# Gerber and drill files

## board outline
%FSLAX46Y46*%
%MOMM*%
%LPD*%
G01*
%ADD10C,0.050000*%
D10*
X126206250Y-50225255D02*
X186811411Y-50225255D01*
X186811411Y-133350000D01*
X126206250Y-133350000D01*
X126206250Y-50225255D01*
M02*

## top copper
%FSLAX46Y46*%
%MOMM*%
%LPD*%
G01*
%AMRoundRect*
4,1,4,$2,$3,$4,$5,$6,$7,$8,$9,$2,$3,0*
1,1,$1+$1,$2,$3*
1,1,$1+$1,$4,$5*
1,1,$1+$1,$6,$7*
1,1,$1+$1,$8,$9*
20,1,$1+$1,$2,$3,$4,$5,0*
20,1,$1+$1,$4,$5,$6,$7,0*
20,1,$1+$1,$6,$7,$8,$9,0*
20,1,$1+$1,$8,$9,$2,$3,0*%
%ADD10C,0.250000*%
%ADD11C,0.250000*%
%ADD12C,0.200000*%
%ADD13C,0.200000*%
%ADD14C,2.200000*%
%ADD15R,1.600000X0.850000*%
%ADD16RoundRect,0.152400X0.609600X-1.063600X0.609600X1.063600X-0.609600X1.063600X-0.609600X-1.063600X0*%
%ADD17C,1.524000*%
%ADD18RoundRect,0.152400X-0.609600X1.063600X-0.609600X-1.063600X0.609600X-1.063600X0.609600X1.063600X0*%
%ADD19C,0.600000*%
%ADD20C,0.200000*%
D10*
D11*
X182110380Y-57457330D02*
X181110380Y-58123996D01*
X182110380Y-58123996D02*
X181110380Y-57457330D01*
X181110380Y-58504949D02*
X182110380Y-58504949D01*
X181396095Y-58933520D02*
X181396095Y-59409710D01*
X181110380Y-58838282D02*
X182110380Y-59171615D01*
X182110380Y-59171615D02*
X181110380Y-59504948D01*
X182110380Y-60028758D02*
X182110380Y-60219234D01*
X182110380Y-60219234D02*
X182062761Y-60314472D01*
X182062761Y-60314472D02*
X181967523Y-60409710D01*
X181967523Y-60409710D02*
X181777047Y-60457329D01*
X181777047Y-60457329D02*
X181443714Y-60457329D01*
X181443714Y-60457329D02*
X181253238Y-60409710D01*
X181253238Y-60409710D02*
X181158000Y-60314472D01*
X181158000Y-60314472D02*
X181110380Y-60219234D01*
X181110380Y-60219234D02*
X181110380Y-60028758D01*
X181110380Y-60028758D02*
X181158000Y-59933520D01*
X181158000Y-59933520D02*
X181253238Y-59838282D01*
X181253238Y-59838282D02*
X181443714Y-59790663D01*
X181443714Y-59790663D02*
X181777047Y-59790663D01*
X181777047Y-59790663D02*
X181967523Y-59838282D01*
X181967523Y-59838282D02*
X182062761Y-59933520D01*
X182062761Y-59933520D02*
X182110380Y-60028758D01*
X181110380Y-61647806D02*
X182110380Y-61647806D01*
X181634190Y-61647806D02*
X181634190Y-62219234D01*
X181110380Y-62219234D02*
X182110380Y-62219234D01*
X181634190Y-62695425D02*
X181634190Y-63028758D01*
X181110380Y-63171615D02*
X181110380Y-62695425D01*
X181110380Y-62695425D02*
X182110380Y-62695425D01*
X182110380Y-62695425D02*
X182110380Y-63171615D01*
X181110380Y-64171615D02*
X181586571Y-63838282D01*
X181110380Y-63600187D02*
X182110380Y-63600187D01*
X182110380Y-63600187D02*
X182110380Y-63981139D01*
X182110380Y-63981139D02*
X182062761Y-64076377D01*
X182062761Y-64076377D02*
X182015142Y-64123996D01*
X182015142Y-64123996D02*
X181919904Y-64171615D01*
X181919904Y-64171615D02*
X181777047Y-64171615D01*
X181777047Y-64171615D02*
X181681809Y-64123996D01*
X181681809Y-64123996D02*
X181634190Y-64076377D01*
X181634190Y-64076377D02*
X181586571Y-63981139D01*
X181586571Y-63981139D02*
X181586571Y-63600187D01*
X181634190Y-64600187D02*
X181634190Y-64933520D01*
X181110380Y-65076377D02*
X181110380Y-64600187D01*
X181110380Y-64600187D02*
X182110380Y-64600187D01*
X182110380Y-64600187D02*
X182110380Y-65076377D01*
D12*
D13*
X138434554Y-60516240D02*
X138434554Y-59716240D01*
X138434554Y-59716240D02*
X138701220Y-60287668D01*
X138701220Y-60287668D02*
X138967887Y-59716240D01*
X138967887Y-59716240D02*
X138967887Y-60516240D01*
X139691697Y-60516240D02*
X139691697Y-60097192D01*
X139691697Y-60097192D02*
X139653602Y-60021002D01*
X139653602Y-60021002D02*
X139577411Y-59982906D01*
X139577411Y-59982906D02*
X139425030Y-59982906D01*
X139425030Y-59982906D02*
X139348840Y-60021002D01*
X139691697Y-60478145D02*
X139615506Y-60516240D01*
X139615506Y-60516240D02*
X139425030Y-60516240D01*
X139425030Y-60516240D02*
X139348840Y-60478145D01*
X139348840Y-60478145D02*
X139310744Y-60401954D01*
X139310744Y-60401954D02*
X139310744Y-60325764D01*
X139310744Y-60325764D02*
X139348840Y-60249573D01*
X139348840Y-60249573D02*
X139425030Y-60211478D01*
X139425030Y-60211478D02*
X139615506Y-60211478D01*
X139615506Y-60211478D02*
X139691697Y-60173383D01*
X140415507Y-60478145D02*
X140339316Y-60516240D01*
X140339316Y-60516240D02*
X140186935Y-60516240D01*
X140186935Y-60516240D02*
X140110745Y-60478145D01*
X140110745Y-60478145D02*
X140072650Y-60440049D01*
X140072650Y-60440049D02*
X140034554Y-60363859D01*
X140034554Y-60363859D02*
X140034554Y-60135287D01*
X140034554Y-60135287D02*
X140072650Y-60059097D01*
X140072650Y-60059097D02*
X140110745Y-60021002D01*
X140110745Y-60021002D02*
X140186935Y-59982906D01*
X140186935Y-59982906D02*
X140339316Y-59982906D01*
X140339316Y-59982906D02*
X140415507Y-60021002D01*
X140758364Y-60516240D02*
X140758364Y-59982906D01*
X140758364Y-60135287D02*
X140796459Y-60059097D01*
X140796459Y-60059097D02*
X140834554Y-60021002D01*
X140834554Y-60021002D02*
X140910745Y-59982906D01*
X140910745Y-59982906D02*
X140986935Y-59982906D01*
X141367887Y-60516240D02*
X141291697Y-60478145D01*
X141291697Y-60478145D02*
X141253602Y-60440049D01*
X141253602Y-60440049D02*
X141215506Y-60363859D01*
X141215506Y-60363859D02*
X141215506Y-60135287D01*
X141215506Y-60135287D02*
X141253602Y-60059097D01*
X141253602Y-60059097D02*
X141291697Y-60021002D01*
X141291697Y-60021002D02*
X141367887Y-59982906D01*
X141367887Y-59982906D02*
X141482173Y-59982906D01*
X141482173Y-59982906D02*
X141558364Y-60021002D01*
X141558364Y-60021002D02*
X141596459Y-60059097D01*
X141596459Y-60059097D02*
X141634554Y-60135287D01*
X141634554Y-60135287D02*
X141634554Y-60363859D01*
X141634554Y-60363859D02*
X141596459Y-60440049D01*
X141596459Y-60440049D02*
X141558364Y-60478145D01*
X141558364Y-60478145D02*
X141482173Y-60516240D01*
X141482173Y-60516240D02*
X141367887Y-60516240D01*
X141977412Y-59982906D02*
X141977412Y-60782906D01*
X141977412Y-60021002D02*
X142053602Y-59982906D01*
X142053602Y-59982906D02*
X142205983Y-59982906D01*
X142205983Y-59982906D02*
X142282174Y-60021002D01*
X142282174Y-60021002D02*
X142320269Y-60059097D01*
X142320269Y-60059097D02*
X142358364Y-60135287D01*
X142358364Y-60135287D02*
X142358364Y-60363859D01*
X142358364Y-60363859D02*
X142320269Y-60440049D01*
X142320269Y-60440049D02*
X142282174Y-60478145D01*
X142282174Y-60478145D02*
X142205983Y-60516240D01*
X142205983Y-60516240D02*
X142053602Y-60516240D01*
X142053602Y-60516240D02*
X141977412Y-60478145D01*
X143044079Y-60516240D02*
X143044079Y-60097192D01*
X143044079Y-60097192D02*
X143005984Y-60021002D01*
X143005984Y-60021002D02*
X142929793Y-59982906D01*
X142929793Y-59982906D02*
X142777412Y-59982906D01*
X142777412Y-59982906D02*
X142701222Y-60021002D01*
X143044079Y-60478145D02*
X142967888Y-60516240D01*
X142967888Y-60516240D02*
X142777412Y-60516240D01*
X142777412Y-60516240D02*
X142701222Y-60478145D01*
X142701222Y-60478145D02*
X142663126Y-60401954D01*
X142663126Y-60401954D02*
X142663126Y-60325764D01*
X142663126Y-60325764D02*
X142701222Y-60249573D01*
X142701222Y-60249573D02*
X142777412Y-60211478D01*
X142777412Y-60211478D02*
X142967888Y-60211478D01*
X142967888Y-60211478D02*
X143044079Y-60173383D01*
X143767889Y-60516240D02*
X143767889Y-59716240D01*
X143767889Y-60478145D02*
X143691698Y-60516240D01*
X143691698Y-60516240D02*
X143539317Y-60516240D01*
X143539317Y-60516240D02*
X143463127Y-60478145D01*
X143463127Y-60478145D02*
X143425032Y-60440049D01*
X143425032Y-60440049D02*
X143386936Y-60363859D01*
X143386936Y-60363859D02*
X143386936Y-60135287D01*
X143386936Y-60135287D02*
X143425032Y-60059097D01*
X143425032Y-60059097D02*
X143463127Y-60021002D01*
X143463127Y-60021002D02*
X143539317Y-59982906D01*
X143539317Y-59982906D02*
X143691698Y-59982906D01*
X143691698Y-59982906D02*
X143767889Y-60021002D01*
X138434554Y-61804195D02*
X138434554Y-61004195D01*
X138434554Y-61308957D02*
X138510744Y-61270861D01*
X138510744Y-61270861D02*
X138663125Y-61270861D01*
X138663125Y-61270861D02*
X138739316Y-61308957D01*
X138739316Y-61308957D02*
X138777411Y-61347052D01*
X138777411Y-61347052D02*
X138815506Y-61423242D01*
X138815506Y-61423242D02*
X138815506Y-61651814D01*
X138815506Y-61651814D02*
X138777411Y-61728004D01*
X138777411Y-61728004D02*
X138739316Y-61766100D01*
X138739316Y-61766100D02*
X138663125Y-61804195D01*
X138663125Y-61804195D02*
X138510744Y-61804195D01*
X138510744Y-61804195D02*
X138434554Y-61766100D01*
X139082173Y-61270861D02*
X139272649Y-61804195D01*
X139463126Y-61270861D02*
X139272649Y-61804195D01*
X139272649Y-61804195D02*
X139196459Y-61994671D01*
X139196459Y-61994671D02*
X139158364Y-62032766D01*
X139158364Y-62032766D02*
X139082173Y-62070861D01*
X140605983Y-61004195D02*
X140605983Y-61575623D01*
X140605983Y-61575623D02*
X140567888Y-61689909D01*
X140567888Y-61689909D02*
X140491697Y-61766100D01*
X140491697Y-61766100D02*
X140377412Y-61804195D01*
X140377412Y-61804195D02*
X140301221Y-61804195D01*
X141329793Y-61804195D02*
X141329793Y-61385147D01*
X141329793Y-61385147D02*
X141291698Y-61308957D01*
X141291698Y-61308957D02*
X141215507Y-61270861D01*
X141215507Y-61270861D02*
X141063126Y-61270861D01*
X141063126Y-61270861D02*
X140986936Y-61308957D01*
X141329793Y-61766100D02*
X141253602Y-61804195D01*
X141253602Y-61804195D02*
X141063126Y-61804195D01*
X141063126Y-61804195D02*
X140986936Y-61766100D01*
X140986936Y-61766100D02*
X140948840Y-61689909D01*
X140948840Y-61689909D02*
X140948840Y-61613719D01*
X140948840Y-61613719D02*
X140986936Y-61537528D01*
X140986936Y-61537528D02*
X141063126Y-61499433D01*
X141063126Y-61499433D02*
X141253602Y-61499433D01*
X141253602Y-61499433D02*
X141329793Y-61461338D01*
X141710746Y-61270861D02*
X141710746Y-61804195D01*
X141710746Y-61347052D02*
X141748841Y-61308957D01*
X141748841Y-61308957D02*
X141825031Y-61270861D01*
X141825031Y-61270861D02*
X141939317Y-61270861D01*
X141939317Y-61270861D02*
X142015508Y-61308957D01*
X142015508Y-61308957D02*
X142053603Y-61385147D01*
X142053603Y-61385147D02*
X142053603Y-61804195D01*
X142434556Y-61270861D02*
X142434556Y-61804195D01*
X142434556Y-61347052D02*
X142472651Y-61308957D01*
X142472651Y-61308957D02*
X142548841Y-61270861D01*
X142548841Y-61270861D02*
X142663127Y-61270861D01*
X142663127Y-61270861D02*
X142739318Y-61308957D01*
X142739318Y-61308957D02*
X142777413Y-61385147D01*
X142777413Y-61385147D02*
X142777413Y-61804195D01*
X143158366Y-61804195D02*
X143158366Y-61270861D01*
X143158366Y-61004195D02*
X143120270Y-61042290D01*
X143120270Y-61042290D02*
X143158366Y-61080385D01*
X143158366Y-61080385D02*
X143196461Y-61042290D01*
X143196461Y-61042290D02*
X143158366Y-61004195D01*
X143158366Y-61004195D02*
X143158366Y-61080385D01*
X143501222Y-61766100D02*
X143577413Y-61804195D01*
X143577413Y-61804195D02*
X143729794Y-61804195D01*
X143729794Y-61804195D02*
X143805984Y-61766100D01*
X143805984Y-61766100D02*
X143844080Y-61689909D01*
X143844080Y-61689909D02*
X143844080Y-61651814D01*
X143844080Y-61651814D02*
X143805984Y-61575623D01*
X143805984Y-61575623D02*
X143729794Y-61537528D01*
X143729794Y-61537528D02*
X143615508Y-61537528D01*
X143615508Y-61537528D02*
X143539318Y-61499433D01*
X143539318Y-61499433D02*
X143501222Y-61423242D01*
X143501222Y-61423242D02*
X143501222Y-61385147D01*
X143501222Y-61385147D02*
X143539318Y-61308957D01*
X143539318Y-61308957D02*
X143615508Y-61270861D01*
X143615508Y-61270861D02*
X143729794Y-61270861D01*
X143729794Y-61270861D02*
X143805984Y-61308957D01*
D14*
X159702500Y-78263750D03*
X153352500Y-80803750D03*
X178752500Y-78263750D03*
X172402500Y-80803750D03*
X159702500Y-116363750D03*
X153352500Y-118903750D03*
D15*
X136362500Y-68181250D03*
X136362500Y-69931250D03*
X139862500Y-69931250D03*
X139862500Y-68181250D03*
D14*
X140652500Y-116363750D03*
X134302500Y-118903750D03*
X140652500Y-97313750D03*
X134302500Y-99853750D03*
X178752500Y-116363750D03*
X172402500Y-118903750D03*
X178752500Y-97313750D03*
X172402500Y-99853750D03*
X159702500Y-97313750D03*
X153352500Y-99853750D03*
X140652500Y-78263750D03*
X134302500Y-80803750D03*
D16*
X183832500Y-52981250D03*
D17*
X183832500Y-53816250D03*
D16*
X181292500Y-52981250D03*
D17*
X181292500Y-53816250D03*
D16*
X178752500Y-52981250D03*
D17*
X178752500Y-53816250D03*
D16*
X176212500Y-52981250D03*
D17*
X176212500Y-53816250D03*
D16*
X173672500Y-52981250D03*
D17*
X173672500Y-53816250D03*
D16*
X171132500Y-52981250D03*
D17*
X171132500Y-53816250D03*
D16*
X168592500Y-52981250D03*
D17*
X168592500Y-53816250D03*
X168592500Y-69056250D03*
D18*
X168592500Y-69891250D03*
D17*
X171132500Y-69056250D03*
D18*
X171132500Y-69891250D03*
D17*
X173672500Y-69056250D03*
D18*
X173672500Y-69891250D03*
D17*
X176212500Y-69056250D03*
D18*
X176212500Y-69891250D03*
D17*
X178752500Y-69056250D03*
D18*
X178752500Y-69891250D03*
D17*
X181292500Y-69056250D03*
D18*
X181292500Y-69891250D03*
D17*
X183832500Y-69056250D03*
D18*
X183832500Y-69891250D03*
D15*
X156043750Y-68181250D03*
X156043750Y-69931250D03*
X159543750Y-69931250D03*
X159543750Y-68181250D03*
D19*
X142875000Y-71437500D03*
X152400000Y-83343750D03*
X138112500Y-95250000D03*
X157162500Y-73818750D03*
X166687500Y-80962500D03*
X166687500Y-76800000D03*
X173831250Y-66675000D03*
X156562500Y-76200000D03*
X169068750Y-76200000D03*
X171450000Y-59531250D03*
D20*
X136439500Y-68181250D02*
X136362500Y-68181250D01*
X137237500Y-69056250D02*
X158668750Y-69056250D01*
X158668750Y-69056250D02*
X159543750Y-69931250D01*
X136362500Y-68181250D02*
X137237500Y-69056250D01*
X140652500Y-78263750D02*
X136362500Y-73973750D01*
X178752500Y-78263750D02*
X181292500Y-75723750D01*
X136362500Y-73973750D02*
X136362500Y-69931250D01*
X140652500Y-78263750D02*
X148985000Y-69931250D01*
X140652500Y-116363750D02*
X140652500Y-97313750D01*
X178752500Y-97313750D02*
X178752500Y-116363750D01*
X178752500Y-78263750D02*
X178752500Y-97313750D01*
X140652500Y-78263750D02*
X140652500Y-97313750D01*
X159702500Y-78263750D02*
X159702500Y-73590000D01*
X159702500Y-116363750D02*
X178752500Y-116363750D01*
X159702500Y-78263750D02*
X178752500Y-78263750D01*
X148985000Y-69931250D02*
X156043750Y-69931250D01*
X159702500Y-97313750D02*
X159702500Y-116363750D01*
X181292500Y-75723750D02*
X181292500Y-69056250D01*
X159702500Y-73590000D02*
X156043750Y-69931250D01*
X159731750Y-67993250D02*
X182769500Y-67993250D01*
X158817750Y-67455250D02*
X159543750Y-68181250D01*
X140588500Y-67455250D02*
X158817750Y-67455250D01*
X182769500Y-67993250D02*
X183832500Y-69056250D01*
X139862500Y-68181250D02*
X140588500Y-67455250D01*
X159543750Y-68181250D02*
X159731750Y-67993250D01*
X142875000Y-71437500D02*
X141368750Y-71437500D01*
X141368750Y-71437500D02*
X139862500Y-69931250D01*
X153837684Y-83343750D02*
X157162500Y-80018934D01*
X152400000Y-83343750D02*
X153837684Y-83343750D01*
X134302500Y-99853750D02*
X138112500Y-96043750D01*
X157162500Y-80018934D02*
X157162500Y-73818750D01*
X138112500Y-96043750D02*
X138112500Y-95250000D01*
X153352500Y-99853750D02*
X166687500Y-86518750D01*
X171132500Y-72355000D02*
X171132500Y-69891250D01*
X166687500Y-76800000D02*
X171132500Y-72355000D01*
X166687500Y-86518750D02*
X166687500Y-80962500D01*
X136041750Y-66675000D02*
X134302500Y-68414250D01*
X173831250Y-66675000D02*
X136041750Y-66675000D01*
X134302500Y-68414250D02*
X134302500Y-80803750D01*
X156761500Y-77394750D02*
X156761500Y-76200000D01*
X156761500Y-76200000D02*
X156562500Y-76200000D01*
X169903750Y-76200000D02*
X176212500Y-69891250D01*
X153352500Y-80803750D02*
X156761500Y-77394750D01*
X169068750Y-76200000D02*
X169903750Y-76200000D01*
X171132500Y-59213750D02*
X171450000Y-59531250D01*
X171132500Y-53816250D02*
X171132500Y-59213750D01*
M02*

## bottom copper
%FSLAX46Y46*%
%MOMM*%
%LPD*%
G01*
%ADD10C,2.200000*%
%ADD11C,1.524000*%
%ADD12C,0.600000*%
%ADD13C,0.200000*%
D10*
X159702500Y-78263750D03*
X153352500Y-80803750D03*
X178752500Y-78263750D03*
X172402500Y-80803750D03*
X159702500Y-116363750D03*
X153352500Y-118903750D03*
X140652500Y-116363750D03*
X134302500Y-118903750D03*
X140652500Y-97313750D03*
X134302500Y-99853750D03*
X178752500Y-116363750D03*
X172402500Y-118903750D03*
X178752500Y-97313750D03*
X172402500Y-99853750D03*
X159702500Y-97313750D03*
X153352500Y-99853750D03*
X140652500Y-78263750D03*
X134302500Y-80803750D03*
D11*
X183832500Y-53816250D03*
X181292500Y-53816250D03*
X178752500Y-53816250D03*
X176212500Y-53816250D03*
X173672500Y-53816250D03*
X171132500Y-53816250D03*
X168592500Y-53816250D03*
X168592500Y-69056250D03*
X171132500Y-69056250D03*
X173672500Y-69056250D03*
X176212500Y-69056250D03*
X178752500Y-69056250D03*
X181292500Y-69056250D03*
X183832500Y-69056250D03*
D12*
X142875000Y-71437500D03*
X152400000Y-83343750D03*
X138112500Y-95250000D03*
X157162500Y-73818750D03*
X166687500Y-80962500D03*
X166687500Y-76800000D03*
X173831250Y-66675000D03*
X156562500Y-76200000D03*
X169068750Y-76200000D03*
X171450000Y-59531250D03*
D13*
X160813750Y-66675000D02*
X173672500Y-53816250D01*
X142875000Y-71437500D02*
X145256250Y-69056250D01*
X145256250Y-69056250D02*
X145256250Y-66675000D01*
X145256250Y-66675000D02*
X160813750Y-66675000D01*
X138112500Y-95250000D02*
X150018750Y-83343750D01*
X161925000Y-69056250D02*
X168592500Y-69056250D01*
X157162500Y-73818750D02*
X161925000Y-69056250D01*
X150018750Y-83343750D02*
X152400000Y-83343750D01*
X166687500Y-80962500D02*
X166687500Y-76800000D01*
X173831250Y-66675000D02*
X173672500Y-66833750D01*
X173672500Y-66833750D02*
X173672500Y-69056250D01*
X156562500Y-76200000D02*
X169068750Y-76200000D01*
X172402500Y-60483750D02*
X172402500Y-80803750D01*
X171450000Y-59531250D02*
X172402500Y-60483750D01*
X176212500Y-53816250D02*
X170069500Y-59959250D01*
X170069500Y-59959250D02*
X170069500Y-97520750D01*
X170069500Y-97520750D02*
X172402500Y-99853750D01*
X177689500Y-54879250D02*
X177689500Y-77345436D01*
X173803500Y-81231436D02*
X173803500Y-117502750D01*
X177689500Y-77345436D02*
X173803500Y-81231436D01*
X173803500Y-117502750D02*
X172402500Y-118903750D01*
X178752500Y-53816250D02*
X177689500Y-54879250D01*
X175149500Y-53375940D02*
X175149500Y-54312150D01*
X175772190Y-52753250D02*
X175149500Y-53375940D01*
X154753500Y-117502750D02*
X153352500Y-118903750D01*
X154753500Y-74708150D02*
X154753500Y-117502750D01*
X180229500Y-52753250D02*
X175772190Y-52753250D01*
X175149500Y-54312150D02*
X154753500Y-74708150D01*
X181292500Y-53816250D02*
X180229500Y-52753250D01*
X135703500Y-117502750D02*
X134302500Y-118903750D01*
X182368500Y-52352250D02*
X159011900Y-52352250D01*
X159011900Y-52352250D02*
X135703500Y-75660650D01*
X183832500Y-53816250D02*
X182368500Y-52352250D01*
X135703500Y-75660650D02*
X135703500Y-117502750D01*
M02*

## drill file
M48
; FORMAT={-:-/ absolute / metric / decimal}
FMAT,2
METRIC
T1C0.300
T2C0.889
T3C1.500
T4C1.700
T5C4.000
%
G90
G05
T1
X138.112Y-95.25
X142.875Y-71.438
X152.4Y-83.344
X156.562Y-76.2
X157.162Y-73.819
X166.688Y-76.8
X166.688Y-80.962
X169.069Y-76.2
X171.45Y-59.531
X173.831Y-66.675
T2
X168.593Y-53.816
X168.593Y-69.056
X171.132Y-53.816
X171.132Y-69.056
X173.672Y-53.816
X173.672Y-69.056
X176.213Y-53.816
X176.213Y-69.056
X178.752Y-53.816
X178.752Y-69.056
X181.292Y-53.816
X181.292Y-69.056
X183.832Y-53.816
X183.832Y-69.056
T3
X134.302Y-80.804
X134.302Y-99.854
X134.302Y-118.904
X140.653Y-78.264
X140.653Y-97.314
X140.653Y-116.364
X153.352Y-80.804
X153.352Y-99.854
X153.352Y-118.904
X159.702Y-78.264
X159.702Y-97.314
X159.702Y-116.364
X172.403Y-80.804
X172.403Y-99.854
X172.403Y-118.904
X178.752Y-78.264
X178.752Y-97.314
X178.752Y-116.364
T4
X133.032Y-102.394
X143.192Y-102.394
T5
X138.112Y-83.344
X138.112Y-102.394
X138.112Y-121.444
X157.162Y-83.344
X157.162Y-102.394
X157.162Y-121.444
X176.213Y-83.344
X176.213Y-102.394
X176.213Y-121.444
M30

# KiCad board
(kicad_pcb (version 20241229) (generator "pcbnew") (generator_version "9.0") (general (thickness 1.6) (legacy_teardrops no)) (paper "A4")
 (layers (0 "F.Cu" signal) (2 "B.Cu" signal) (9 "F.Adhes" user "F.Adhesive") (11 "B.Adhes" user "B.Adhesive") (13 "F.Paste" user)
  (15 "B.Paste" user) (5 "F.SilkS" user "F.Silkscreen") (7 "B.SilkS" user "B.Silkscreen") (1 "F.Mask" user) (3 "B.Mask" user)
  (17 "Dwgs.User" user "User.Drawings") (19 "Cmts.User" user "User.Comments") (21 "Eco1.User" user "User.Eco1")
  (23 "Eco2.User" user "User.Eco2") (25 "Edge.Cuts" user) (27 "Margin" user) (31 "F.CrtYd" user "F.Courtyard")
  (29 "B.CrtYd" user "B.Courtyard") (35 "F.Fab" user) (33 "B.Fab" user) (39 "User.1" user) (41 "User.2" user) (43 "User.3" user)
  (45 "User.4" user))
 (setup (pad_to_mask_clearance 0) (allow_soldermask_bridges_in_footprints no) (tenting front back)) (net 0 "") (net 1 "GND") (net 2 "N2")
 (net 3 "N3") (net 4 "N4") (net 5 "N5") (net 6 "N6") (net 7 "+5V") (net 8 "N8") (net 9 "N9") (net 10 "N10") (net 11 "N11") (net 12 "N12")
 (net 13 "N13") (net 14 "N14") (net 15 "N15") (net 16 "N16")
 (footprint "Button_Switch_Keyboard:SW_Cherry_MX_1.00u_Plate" (layer "F.Cu") (at 159.7025 78.26375)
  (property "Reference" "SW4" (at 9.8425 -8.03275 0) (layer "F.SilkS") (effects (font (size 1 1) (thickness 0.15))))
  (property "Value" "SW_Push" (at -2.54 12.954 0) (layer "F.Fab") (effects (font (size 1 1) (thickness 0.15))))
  (pad "" np_thru_hole circle (at -2.54 5.08) (size 4 4) (drill 4) (layers "*.Cu" "*.Mask"))
  (pad "1" thru_hole circle (at 0 0) (size 2.2 2.2) (drill 1.5) (layers "*.Cu" "*.Mask") (remove_unused_layers no) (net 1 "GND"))
  (pad "2" thru_hole circle (at -6.35 2.54) (size 2.2 2.2) (drill 1.5) (layers "*.Cu" "*.Mask") (remove_unused_layers no) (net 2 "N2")))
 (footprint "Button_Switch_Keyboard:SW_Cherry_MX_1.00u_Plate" (layer "F.Cu") (at 178.7525 78.26375)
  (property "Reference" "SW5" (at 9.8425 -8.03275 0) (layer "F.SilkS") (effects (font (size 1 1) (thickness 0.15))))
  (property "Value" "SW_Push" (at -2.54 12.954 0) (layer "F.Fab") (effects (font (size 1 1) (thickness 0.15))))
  (pad "" np_thru_hole circle (at -2.54 5.08) (size 4 4) (drill 4) (layers "*.Cu" "*.Mask"))
  (pad "1" thru_hole circle (at 0 0) (size 2.2 2.2) (drill 1.5) (layers "*.Cu" "*.Mask") (remove_unused_layers no) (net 1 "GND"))
  (pad "2" thru_hole circle (at -6.35 2.54) (size 2.2 2.2) (drill 1.5) (layers "*.Cu" "*.Mask") (remove_unused_layers no) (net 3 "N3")))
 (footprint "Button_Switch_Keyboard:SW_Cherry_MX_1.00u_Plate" (layer "F.Cu") (at 159.7025 116.36375)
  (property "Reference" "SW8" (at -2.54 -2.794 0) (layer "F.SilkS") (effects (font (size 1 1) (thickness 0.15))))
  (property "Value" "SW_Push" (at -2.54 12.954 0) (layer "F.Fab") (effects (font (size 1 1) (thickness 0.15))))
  (pad "" np_thru_hole circle (at -2.54 5.08) (size 4 4) (drill 4) (layers "*.Cu" "*.Mask"))
  (pad "1" thru_hole circle (at 0 0) (size 2.2 2.2) (drill 1.5) (layers "*.Cu" "*.Mask") (remove_unused_layers no) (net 1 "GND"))
  (pad "2" thru_hole circle (at -6.35 2.54) (size 2.2 2.2) (drill 1.5) (layers "*.Cu" "*.Mask") (remove_unused_layers no) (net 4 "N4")))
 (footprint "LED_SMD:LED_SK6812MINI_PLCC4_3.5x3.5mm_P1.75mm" (layer "F.Cu") (at 138.1125 69.05625)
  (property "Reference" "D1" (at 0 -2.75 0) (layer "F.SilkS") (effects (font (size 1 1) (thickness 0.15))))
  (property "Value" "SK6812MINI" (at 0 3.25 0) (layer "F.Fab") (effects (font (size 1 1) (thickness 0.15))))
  (pad "1" smd rect (at -1.75 -0.875) (size 1.6 0.85) (layers "F.Cu" "F.Mask" "F.Paste") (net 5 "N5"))
  (pad "2" smd rect (at -1.75 0.875) (size 1.6 0.85) (layers "F.Cu" "F.Mask" "F.Paste") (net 1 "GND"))
  (pad "3" smd rect (at 1.75 0.875) (size 1.6 0.85) (layers "F.Cu" "F.Mask" "F.Paste") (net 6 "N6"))
  (pad "4" smd rect (at 1.75 -0.875) (size 1.6 0.85) (layers "F.Cu" "F.Mask" "F.Paste") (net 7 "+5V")))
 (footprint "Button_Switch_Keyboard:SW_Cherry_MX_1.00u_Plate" (layer "F.Cu") (at 140.6525 116.36375)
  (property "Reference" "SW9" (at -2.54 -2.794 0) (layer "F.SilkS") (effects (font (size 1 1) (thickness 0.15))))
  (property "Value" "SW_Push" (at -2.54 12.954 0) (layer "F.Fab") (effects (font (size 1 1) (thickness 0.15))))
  (pad "" np_thru_hole circle (at -2.54 5.08) (size 4 4) (drill 4) (layers "*.Cu" "*.Mask"))
  (pad "1" thru_hole circle (at 0 0) (size 2.2 2.2) (drill 1.5) (layers "*.Cu" "*.Mask") (remove_unused_layers no) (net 1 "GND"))
  (pad "2" thru_hole circle (at -6.35 2.54) (size 2.2 2.2) (drill 1.5) (layers "*.Cu" "*.Mask") (remove_unused_layers no) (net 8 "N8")))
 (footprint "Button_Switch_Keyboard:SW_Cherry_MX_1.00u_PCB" (layer "F.Cu") (at 140.6525 97.31375)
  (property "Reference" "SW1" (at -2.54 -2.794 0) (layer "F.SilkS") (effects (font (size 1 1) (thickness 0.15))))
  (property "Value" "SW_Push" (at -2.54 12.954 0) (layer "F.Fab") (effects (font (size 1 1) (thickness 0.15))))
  (pad "" np_thru_hole circle (at -7.62 5.08) (size 1.7 1.7) (drill 1.7) (layers "*.Cu" "*.Mask"))
  (pad "" np_thru_hole circle (at -2.54 5.08) (size 4 4) (drill 4) (layers "*.Cu" "*.Mask"))
  (pad "" np_thru_hole circle (at 2.54 5.08) (size 1.7 1.7) (drill 1.7) (layers "*.Cu" "*.Mask"))
  (pad "1" thru_hole circle (at 0 0) (size 2.2 2.2) (drill 1.5) (layers "*.Cu" "*.Mask") (remove_unused_layers no) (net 1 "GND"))
  (pad "2" thru_hole circle (at -6.35 2.54) (size 2.2 2.2) (drill 1.5) (layers "*.Cu" "*.Mask") (remove_unused_layers no) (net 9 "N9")))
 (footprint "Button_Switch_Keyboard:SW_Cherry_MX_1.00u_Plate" (layer "F.Cu") (at 178.7525 116.36375)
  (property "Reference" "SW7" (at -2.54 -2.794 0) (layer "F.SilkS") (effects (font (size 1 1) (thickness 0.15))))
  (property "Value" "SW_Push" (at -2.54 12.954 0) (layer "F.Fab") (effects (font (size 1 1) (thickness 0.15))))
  (pad "" np_thru_hole circle (at -2.54 5.08) (size 4 4) (drill 4) (layers "*.Cu" "*.Mask"))
  (pad "1" thru_hole circle (at 0 0) (size 2.2 2.2) (drill 1.5) (layers "*.Cu" "*.Mask") (remove_unused_layers no) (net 1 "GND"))
  (pad "2" thru_hole circle (at -6.35 2.54) (size 2.2 2.2) (drill 1.5) (layers "*.Cu" "*.Mask") (remove_unused_layers no) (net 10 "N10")))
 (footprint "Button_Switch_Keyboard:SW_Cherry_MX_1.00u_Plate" (layer "F.Cu") (at 178.7525 97.31375)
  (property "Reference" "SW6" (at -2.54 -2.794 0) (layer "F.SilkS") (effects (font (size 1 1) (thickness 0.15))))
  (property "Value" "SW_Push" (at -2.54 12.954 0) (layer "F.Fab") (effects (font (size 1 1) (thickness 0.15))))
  (pad "" np_thru_hole circle (at -2.54 5.08) (size 4 4) (drill 4) (layers "*.Cu" "*.Mask"))
  (pad "1" thru_hole circle (at 0 0) (size 2.2 2.2) (drill 1.5) (layers "*.Cu" "*.Mask") (remove_unused_layers no) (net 1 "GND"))
  (pad "2" thru_hole circle (at -6.35 2.54) (size 2.2 2.2) (drill 1.5) (layers "*.Cu" "*.Mask") (remove_unused_layers no) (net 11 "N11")))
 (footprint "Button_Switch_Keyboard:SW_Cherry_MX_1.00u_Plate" (layer "F.Cu") (at 159.7025 97.31375)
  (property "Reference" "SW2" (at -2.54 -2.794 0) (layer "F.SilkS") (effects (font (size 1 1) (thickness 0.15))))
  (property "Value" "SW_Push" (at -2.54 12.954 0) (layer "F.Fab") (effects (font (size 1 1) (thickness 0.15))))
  (pad "" np_thru_hole circle (at -2.54 5.08) (size 4 4) (drill 4) (layers "*.Cu" "*.Mask"))
  (pad "1" thru_hole circle (at 0 0) (size 2.2 2.2) (drill 1.5) (layers "*.Cu" "*.Mask") (remove_unused_layers no) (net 1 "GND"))
  (pad "2" thru_hole circle (at -6.35 2.54) (size 2.2 2.2) (drill 1.5) (layers "*.Cu" "*.Mask") (remove_unused_layers no) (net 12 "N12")))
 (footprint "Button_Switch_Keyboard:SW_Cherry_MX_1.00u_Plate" (layer "F.Cu") (at 140.6525 78.26375)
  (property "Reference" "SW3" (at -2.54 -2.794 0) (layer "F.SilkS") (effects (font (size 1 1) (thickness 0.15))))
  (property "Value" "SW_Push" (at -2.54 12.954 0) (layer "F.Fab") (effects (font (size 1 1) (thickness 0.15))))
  (pad "" np_thru_hole circle (at -2.54 5.08) (size 4 4) (drill 4) (layers "*.Cu" "*.Mask"))
  (pad "1" thru_hole circle (at 0 0) (size 2.2 2.2) (drill 1.5) (layers "*.Cu" "*.Mask") (remove_unused_layers no) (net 1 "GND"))
  (pad "2" thru_hole circle (at -6.35 2.54) (size 2.2 2.2) (drill 1.5) (layers "*.Cu" "*.Mask") (remove_unused_layers no) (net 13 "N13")))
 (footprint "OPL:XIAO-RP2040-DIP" (layer "F.Cu") (at 176.2125 61.43625 -90)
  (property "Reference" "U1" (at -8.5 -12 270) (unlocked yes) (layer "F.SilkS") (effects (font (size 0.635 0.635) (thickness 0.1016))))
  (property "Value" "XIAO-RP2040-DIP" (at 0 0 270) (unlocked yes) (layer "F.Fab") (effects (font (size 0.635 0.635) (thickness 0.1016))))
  (pad "1" smd roundrect (at -8.455 -7.62 90) (size 2.432 1.524) (layers "F.Cu" "F.Mask") (roundrect_rratio 0.1) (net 8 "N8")
   (thermal_bridge_angle 45))
  (pad "1" thru_hole circle (at -7.62 -7.62 90) (size 1.524 1.524) (drill 0.889) (layers "*.Cu" "*.Mask") (remove_unused_layers no)
   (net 8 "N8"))
  (pad "2" smd roundrect (at -8.455 -5.08 90) (size 2.432 1.524) (layers "F.Cu" "F.Mask") (roundrect_rratio 0.1) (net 4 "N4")
   (thermal_bridge_angle 45))
  (pad "2" thru_hole circle (at -7.62 -5.08 90) (size 1.524 1.524) (drill 0.889) (layers "*.Cu" "*.Mask") (remove_unused_layers no)
   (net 4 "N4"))
  (pad "3" smd roundrect (at -8.455 -2.54 90) (size 2.432 1.524) (layers "F.Cu" "F.Mask") (roundrect_rratio 0.1) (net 10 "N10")
   (thermal_bridge_angle 45))
  (pad "3" thru_hole circle (at -7.62 -2.54 90) (size 1.524 1.524) (drill 0.889) (layers "*.Cu" "*.Mask") (remove_unused_layers no)
   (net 10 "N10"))
  (pad "4" smd roundrect (at -8.455 0 90) (size 2.432 1.524) (layers "F.Cu" "F.Mask") (roundrect_rratio 0.1) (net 11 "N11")
   (thermal_bridge_angle 45))
  (pad "4" thru_hole circle (at -7.62 0 90) (size 1.524 1.524) (drill 0.889) (layers "*.Cu" "*.Mask") (remove_unused_layers no)
   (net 11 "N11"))
  (pad "5" smd roundrect (at -8.455 2.54 90) (size 2.432 1.524) (layers "F.Cu" "F.Mask") (roundrect_rratio 0.1) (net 6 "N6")
   (thermal_bridge_angle 45))
  (pad "5" thru_hole circle (at -7.62 2.54 90) (size 1.524 1.524) (drill 0.889) (layers "*.Cu" "*.Mask") (remove_unused_layers no)
   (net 6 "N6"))
  (pad "6" smd roundrect (at -8.455 5.08 90) (size 2.432 1.524) (layers "F.Cu" "F.Mask") (roundrect_rratio 0.1) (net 3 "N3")
   (thermal_bridge_angle 45))
  (pad "6" thru_hole circle (at -7.62 5.08 90) (size 1.524 1.524) (drill 0.889) (layers "*.Cu" "*.Mask") (remove_unused_layers no)
   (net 3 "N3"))
  (pad "7" smd roundrect (at -8.455 7.62 90) (size 2.432 1.524) (layers "F.Cu" "F.Mask") (roundrect_rratio 0.1) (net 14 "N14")
   (thermal_bridge_angle 45))
  (pad "7" thru_hole circle (at -7.62 7.62 90) (size 1.524 1.524) (drill 0.889) (layers "*.Cu" "*.Mask") (remove_unused_layers no)
   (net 14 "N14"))
  (pad "8" thru_hole circle (at 7.62 7.62 270) (size 1.524 1.524) (drill 0.889) (layers "*.Cu" "*.Mask") (remove_unused_layers no)
   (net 9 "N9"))
  (pad "8" smd roundrect (at 8.455 7.62 270) (size 2.432 1.524) (layers "F.Cu" "F.Mask") (roundrect_rratio 0.1) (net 9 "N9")
   (thermal_bridge_angle 45))
  (pad "9" thru_hole circle (at 7.62 5.08 270) (size 1.524 1.524) (drill 0.889) (layers "*.Cu" "*.Mask") (remove_unused_layers no)
   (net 12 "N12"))
  (pad "9" smd roundrect (at 8.455 5.08 270) (size 2.432 1.524) (layers "F.Cu" "F.Mask") (roundrect_rratio 0.1) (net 12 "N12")
   (thermal_bridge_angle 45))
  (pad "10" thru_hole circle (at 7.62 2.54 270) (size 1.524 1.524) (drill 0.889) (layers "*.Cu" "*.Mask") (remove_unused_layers no)
   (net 13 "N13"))
  (pad "10" smd roundrect (at 8.455 2.54 270) (size 2.432 1.524) (layers "F.Cu" "F.Mask") (roundrect_rratio 0.1) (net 13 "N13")
   (thermal_bridge_angle 45))
  (pad "11" thru_hole circle (at 7.62 0 270) (size 1.524 1.524) (drill 0.889) (layers "*.Cu" "*.Mask") (remove_unused_layers no)
   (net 2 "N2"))
  (pad "11" smd roundrect (at 8.455 0 270) (size 2.432 1.524) (layers "F.Cu" "F.Mask") (roundrect_rratio 0.1) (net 2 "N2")
   (thermal_bridge_angle 45))
  (pad "12" thru_hole circle (at 7.62 -2.54 270) (size 1.524 1.524) (drill 0.889) (layers "*.Cu" "*.Mask") (remove_unused_layers no)
   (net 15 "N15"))
  (pad "12" smd roundrect (at 8.455 -2.54 270) (size 2.432 1.524) (layers "F.Cu" "F.Mask") (roundrect_rratio 0.1) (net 15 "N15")
   (thermal_bridge_angle 45))
  (pad "13" thru_hole circle (at 7.62 -5.08 270) (size 1.524 1.524) (drill 0.889) (layers "*.Cu" "*.Mask") (remove_unused_layers no)
   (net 1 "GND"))
  (pad "13" smd roundrect (at 8.455 -5.08 270) (size 2.432 1.524) (layers "F.Cu" "F.Mask") (roundrect_rratio 0.1) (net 1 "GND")
   (thermal_bridge_angle 45))
  (pad "14" thru_hole circle (at 7.62 -7.62 270) (size 1.524 1.524) (drill 0.889) (layers "*.Cu" "*.Mask") (remove_unused_layers no)
   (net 7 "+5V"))
  (pad "14" smd roundrect (at 8.455 -7.62 270) (size 2.432 1.524) (layers "F.Cu" "F.Mask") (roundrect_rratio 0.1) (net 7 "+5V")
   (thermal_bridge_angle 45)))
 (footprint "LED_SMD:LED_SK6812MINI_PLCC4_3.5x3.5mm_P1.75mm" (layer "F.Cu") (at 157.79375 69.05625)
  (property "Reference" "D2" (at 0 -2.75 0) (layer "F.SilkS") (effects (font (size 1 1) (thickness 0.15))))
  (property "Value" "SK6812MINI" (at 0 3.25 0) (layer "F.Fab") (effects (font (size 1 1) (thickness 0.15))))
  (pad "1" smd rect (at -1.75 -0.875) (size 1.6 0.85) (layers "F.Cu" "F.Mask" "F.Paste") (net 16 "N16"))
  (pad "2" smd rect (at -1.75 0.875) (size 1.6 0.85) (layers "F.Cu" "F.Mask" "F.Paste") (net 1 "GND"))
  (pad "3" smd rect (at 1.75 0.875) (size 1.6 0.85) (layers "F.Cu" "F.Mask" "F.Paste") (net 5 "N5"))
  (pad "4" smd rect (at 1.75 -0.875) (size 1.6 0.85) (layers "F.Cu" "F.Mask" "F.Paste") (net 7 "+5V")))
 (gr_rect (start 126.20625 50.225255) (end 186.811411 133.35) (stroke (width 0.05) (type default)) (fill no) (layer "Edge.Cuts"))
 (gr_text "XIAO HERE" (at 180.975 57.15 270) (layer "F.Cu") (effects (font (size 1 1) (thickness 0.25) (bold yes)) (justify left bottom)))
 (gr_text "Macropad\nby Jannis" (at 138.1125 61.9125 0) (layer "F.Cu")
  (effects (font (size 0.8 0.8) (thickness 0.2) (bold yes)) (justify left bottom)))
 (segment (start 136.4395 68.18125) (end 136.3625 68.18125) (width 0.2) (layer "F.Cu") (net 5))
 (segment (start 137.2375 69.05625) (end 158.66875 69.05625) (width 0.2) (layer "F.Cu") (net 5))
 (segment (start 158.66875 69.05625) (end 159.54375 69.93125) (width 0.2) (layer "F.Cu") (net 5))
 (segment (start 136.3625 68.18125) (end 137.2375 69.05625) (width 0.2) (layer "F.Cu") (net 5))
 (segment (start 140.6525 78.26375) (end 136.3625 73.97375) (width 0.2) (layer "F.Cu") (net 1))
 (segment (start 178.7525 78.26375) (end 181.2925 75.72375) (width 0.2) (layer "F.Cu") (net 1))
 (segment (start 136.3625 73.97375) (end 136.3625 69.93125) (width 0.2) (layer "F.Cu") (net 1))
 (segment (start 140.6525 78.26375) (end 148.985 69.93125) (width 0.2) (layer "F.Cu") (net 1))
 (segment (start 140.6525 116.36375) (end 140.6525 97.31375) (width 0.2) (layer "F.Cu") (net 1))
 (segment (start 178.7525 97.31375) (end 178.7525 116.36375) (width 0.2) (layer "F.Cu") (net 1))
 (segment (start 178.7525 78.26375) (end 178.7525 97.31375) (width 0.2) (layer "F.Cu") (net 1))
 (segment (start 140.6525 78.26375) (end 140.6525 97.31375) (width 0.2) (layer "F.Cu") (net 1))
 (segment (start 159.7025 78.26375) (end 159.7025 73.59) (width 0.2) (layer "F.Cu") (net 1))
 (segment (start 159.7025 116.36375) (end 178.7525 116.36375) (width 0.2) (layer "F.Cu") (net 1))
 (segment (start 159.7025 78.26375) (end 178.7525 78.26375) (width 0.2) (layer "F.Cu") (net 1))
 (segment (start 148.985 69.93125) (end 156.04375 69.93125) (width 0.2) (layer "F.Cu") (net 1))
 (segment (start 159.7025 97.31375) (end 159.7025 116.36375) (width 0.2) (layer "F.Cu") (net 1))
 (segment (start 181.2925 75.72375) (end 181.2925 69.05625) (width 0.2) (layer "F.Cu") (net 1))
 (segment (start 159.7025 73.59) (end 156.04375 69.93125) (width 0.2) (layer "F.Cu") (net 1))
 (segment (start 159.73175 67.99325) (end 182.7695 67.99325) (width 0.2) (layer "F.Cu") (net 7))
 (segment (start 158.81775 67.45525) (end 159.54375 68.18125) (width 0.2) (layer "F.Cu") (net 7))
 (segment (start 140.5885 67.45525) (end 158.81775 67.45525) (width 0.2) (layer "F.Cu") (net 7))
 (segment (start 182.7695 67.99325) (end 183.8325 69.05625) (width 0.2) (layer "F.Cu") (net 7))
 (segment (start 139.8625 68.18125) (end 140.5885 67.45525) (width 0.2) (layer "F.Cu") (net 7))
 (segment (start 159.54375 68.18125) (end 159.73175 67.99325) (width 0.2) (layer "F.Cu") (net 7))
 (segment (start 142.875 71.4375) (end 141.36875 71.4375) (width 0.2) (layer "F.Cu") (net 6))
 (segment (start 141.36875 71.4375) (end 139.8625 69.93125) (width 0.2) (layer "F.Cu") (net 6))
 (via (at 142.875 71.4375) (size 0.6) (drill 0.3) (layers "F.Cu" "B.Cu") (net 6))
 (segment (start 160.81375 66.675) (end 173.6725 53.81625) (width 0.2) (layer "B.Cu") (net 6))
 (segment (start 142.875 71.4375) (end 145.25625 69.05625) (width 0.2) (layer "B.Cu") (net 6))
 (segment (start 145.25625 69.05625) (end 145.25625 66.675) (width 0.2) (layer "B.Cu") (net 6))
 (segment (start 145.25625 66.675) (end 160.81375 66.675) (width 0.2) (layer "B.Cu") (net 6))
 (segment (start 153.837684 83.34375) (end 157.1625 80.018934) (width 0.2) (layer "F.Cu") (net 9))
 (segment (start 152.4 83.34375) (end 153.837684 83.34375) (width 0.2) (layer "F.Cu") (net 9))
 (segment (start 134.3025 99.85375) (end 138.1125 96.04375) (width 0.2) (layer "F.Cu") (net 9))
 (segment (start 157.1625 80.018934) (end 157.1625 73.81875) (width 0.2) (layer "F.Cu") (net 9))
 (segment (start 138.1125 96.04375) (end 138.1125 95.25) (width 0.2) (layer "F.Cu") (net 9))
 (via (at 152.4 83.34375) (size 0.6) (drill 0.3) (layers "F.Cu" "B.Cu") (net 9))
 (via (at 138.1125 95.25) (size 0.6) (drill 0.3) (layers "F.Cu" "B.Cu") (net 9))
 (via (at 157.1625 73.81875) (size 0.6) (drill 0.3) (layers "F.Cu" "B.Cu") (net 9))
 (segment (start 138.1125 95.25) (end 150.01875 83.34375) (width 0.2) (layer "B.Cu") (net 9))
 (segment (start 161.925 69.05625) (end 168.5925 69.05625) (width 0.2) (layer "B.Cu") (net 9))
 (segment (start 157.1625 73.81875) (end 161.925 69.05625) (width 0.2) (layer "B.Cu") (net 9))
 (segment (start 150.01875 83.34375) (end 152.4 83.34375) (width 0.2) (layer "B.Cu") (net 9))
 (segment (start 153.3525 99.85375) (end 166.6875 86.51875) (width 0.2) (layer "F.Cu") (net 12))
 (segment (start 171.1325 72.355) (end 171.1325 69.89125) (width 0.2) (layer "F.Cu") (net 12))
 (segment (start 166.6875 76.8) (end 171.1325 72.355) (width 0.2) (layer "F.Cu") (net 12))
 (segment (start 166.6875 86.51875) (end 166.6875 80.9625) (width 0.2) (layer "F.Cu") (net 12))
 (via (at 166.6875 80.9625) (size 0.6) (drill 0.3) (layers "F.Cu" "B.Cu") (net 12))
 (via (at 166.6875 76.8) (size 0.6) (drill 0.3) (layers "F.Cu" "B.Cu") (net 12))
 (segment (start 166.6875 80.9625) (end 166.6875 76.8) (width 0.2) (layer "B.Cu") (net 12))
 (segment (start 136.04175 66.675) (end 134.3025 68.41425) (width 0.2) (layer "F.Cu") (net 13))
 (segment (start 173.83125 66.675) (end 136.04175 66.675) (width 0.2) (layer "F.Cu") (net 13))
 (segment (start 134.3025 68.41425) (end 134.3025 80.80375) (width 0.2) (layer "F.Cu") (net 13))
 (via (at 173.83125 66.675) (size 0.6) (drill 0.3) (layers "F.Cu" "B.Cu") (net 13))
 (segment (start 173.83125 66.675) (end 173.6725 66.83375) (width 0.2) (layer "B.Cu") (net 13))
 (segment (start 173.6725 66.83375) (end 173.6725 69.05625) (width 0.2) (layer "B.Cu") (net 13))
 (segment (start 156.7615 77.39475) (end 156.7615 76.2) (width 0.2) (layer "F.Cu") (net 2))
 (segment (start 156.7615 76.2) (end 156.5625 76.2) (width 0.2) (layer "F.Cu") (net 2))
 (segment (start 169.90375 76.2) (end 176.2125 69.89125) (width 0.2) (layer "F.Cu") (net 2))
 (segment (start 153.3525 80.80375) (end 156.7615 77.39475) (width 0.2) (layer "F.Cu") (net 2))
 (segment (start 169.06875 76.2) (end 169.90375 76.2) (width 0.2) (layer "F.Cu") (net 2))
 (via (at 156.5625 76.2) (size 0.6) (drill 0.3) (layers "F.Cu" "B.Cu") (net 2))
 (via (at 169.06875 76.2) (size 0.6) (drill 0.3) (layers "F.Cu" "B.Cu") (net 2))
 (segment (start 156.5625 76.2) (end 169.06875 76.2) (width 0.2) (layer "B.Cu") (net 2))
 (segment (start 171.1325 59.21375) (end 171.45 59.53125) (width 0.2) (layer "F.Cu") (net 3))
 (segment (start 171.1325 53.81625) (end 171.1325 59.21375) (width 0.2) (layer "F.Cu") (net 3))
 (via (at 171.45 59.53125) (size 0.6) (drill 0.3) (layers "F.Cu" "B.Cu") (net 3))
 (segment (start 172.4025 60.48375) (end 172.4025 80.80375) (width 0.2) (layer "B.Cu") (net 3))
 (segment (start 171.45 59.53125) (end 172.4025 60.48375) (width 0.2) (layer "B.Cu") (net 3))
 (segment (start 176.2125 53.81625) (end 170.0695 59.95925) (width 0.2) (layer "B.Cu") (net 11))
 (segment (start 170.0695 59.95925) (end 170.0695 97.52075) (width 0.2) (layer "B.Cu") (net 11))
 (segment (start 170.0695 97.52075) (end 172.4025 99.85375) (width 0.2) (layer "B.Cu") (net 11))
 (segment (start 177.6895 54.87925) (end 177.6895 77.345436) (width 0.2) (layer "B.Cu") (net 10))
 (segment (start 173.8035 81.231436) (end 173.8035 117.50275) (width 0.2) (layer "B.Cu") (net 10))
 (segment (start 177.6895 77.345436) (end 173.8035 81.231436) (width 0.2) (layer "B.Cu") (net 10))
 (segment (start 173.8035 117.50275) (end 172.4025 118.90375) (width 0.2) (layer "B.Cu") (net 10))
 (segment (start 178.7525 53.81625) (end 177.6895 54.87925) (width 0.2) (layer "B.Cu") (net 10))
 (segment (start 175.1495 53.37594) (end 175.1495 54.31215) (width 0.2) (layer "B.Cu") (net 4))
 (segment (start 175.77219 52.75325) (end 175.1495 53.37594) (width 0.2) (layer "B.Cu") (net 4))
 (segment (start 154.7535 117.50275) (end 153.3525 118.90375) (width 0.2) (layer "B.Cu") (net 4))
 (segment (start 154.7535 74.70815) (end 154.7535 117.50275) (width 0.2) (layer "B.Cu") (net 4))
 (segment (start 180.2295 52.75325) (end 175.77219 52.75325) (width 0.2) (layer "B.Cu") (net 4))
 (segment (start 175.1495 54.31215) (end 154.7535 74.70815) (width 0.2) (layer "B.Cu") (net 4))
 (segment (start 181.2925 53.81625) (end 180.2295 52.75325) (width 0.2) (layer "B.Cu") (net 4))
 (segment (start 135.7035 117.50275) (end 134.3025 118.90375) (width 0.2) (layer "B.Cu") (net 8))
 (segment (start 182.3685 52.35225) (end 159.0119 52.35225) (width 0.2) (layer "B.Cu") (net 8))
 (segment (start 159.0119 52.35225) (end 135.7035 75.66065) (width 0.2) (layer "B.Cu") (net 8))
 (segment (start 183.8325 53.81625) (end 182.3685 52.35225) (width 0.2) (layer "B.Cu") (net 8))
 (segment (start 135.7035 75.66065) (end 135.7035 117.50275) (width 0.2) (layer "B.Cu") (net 8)))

